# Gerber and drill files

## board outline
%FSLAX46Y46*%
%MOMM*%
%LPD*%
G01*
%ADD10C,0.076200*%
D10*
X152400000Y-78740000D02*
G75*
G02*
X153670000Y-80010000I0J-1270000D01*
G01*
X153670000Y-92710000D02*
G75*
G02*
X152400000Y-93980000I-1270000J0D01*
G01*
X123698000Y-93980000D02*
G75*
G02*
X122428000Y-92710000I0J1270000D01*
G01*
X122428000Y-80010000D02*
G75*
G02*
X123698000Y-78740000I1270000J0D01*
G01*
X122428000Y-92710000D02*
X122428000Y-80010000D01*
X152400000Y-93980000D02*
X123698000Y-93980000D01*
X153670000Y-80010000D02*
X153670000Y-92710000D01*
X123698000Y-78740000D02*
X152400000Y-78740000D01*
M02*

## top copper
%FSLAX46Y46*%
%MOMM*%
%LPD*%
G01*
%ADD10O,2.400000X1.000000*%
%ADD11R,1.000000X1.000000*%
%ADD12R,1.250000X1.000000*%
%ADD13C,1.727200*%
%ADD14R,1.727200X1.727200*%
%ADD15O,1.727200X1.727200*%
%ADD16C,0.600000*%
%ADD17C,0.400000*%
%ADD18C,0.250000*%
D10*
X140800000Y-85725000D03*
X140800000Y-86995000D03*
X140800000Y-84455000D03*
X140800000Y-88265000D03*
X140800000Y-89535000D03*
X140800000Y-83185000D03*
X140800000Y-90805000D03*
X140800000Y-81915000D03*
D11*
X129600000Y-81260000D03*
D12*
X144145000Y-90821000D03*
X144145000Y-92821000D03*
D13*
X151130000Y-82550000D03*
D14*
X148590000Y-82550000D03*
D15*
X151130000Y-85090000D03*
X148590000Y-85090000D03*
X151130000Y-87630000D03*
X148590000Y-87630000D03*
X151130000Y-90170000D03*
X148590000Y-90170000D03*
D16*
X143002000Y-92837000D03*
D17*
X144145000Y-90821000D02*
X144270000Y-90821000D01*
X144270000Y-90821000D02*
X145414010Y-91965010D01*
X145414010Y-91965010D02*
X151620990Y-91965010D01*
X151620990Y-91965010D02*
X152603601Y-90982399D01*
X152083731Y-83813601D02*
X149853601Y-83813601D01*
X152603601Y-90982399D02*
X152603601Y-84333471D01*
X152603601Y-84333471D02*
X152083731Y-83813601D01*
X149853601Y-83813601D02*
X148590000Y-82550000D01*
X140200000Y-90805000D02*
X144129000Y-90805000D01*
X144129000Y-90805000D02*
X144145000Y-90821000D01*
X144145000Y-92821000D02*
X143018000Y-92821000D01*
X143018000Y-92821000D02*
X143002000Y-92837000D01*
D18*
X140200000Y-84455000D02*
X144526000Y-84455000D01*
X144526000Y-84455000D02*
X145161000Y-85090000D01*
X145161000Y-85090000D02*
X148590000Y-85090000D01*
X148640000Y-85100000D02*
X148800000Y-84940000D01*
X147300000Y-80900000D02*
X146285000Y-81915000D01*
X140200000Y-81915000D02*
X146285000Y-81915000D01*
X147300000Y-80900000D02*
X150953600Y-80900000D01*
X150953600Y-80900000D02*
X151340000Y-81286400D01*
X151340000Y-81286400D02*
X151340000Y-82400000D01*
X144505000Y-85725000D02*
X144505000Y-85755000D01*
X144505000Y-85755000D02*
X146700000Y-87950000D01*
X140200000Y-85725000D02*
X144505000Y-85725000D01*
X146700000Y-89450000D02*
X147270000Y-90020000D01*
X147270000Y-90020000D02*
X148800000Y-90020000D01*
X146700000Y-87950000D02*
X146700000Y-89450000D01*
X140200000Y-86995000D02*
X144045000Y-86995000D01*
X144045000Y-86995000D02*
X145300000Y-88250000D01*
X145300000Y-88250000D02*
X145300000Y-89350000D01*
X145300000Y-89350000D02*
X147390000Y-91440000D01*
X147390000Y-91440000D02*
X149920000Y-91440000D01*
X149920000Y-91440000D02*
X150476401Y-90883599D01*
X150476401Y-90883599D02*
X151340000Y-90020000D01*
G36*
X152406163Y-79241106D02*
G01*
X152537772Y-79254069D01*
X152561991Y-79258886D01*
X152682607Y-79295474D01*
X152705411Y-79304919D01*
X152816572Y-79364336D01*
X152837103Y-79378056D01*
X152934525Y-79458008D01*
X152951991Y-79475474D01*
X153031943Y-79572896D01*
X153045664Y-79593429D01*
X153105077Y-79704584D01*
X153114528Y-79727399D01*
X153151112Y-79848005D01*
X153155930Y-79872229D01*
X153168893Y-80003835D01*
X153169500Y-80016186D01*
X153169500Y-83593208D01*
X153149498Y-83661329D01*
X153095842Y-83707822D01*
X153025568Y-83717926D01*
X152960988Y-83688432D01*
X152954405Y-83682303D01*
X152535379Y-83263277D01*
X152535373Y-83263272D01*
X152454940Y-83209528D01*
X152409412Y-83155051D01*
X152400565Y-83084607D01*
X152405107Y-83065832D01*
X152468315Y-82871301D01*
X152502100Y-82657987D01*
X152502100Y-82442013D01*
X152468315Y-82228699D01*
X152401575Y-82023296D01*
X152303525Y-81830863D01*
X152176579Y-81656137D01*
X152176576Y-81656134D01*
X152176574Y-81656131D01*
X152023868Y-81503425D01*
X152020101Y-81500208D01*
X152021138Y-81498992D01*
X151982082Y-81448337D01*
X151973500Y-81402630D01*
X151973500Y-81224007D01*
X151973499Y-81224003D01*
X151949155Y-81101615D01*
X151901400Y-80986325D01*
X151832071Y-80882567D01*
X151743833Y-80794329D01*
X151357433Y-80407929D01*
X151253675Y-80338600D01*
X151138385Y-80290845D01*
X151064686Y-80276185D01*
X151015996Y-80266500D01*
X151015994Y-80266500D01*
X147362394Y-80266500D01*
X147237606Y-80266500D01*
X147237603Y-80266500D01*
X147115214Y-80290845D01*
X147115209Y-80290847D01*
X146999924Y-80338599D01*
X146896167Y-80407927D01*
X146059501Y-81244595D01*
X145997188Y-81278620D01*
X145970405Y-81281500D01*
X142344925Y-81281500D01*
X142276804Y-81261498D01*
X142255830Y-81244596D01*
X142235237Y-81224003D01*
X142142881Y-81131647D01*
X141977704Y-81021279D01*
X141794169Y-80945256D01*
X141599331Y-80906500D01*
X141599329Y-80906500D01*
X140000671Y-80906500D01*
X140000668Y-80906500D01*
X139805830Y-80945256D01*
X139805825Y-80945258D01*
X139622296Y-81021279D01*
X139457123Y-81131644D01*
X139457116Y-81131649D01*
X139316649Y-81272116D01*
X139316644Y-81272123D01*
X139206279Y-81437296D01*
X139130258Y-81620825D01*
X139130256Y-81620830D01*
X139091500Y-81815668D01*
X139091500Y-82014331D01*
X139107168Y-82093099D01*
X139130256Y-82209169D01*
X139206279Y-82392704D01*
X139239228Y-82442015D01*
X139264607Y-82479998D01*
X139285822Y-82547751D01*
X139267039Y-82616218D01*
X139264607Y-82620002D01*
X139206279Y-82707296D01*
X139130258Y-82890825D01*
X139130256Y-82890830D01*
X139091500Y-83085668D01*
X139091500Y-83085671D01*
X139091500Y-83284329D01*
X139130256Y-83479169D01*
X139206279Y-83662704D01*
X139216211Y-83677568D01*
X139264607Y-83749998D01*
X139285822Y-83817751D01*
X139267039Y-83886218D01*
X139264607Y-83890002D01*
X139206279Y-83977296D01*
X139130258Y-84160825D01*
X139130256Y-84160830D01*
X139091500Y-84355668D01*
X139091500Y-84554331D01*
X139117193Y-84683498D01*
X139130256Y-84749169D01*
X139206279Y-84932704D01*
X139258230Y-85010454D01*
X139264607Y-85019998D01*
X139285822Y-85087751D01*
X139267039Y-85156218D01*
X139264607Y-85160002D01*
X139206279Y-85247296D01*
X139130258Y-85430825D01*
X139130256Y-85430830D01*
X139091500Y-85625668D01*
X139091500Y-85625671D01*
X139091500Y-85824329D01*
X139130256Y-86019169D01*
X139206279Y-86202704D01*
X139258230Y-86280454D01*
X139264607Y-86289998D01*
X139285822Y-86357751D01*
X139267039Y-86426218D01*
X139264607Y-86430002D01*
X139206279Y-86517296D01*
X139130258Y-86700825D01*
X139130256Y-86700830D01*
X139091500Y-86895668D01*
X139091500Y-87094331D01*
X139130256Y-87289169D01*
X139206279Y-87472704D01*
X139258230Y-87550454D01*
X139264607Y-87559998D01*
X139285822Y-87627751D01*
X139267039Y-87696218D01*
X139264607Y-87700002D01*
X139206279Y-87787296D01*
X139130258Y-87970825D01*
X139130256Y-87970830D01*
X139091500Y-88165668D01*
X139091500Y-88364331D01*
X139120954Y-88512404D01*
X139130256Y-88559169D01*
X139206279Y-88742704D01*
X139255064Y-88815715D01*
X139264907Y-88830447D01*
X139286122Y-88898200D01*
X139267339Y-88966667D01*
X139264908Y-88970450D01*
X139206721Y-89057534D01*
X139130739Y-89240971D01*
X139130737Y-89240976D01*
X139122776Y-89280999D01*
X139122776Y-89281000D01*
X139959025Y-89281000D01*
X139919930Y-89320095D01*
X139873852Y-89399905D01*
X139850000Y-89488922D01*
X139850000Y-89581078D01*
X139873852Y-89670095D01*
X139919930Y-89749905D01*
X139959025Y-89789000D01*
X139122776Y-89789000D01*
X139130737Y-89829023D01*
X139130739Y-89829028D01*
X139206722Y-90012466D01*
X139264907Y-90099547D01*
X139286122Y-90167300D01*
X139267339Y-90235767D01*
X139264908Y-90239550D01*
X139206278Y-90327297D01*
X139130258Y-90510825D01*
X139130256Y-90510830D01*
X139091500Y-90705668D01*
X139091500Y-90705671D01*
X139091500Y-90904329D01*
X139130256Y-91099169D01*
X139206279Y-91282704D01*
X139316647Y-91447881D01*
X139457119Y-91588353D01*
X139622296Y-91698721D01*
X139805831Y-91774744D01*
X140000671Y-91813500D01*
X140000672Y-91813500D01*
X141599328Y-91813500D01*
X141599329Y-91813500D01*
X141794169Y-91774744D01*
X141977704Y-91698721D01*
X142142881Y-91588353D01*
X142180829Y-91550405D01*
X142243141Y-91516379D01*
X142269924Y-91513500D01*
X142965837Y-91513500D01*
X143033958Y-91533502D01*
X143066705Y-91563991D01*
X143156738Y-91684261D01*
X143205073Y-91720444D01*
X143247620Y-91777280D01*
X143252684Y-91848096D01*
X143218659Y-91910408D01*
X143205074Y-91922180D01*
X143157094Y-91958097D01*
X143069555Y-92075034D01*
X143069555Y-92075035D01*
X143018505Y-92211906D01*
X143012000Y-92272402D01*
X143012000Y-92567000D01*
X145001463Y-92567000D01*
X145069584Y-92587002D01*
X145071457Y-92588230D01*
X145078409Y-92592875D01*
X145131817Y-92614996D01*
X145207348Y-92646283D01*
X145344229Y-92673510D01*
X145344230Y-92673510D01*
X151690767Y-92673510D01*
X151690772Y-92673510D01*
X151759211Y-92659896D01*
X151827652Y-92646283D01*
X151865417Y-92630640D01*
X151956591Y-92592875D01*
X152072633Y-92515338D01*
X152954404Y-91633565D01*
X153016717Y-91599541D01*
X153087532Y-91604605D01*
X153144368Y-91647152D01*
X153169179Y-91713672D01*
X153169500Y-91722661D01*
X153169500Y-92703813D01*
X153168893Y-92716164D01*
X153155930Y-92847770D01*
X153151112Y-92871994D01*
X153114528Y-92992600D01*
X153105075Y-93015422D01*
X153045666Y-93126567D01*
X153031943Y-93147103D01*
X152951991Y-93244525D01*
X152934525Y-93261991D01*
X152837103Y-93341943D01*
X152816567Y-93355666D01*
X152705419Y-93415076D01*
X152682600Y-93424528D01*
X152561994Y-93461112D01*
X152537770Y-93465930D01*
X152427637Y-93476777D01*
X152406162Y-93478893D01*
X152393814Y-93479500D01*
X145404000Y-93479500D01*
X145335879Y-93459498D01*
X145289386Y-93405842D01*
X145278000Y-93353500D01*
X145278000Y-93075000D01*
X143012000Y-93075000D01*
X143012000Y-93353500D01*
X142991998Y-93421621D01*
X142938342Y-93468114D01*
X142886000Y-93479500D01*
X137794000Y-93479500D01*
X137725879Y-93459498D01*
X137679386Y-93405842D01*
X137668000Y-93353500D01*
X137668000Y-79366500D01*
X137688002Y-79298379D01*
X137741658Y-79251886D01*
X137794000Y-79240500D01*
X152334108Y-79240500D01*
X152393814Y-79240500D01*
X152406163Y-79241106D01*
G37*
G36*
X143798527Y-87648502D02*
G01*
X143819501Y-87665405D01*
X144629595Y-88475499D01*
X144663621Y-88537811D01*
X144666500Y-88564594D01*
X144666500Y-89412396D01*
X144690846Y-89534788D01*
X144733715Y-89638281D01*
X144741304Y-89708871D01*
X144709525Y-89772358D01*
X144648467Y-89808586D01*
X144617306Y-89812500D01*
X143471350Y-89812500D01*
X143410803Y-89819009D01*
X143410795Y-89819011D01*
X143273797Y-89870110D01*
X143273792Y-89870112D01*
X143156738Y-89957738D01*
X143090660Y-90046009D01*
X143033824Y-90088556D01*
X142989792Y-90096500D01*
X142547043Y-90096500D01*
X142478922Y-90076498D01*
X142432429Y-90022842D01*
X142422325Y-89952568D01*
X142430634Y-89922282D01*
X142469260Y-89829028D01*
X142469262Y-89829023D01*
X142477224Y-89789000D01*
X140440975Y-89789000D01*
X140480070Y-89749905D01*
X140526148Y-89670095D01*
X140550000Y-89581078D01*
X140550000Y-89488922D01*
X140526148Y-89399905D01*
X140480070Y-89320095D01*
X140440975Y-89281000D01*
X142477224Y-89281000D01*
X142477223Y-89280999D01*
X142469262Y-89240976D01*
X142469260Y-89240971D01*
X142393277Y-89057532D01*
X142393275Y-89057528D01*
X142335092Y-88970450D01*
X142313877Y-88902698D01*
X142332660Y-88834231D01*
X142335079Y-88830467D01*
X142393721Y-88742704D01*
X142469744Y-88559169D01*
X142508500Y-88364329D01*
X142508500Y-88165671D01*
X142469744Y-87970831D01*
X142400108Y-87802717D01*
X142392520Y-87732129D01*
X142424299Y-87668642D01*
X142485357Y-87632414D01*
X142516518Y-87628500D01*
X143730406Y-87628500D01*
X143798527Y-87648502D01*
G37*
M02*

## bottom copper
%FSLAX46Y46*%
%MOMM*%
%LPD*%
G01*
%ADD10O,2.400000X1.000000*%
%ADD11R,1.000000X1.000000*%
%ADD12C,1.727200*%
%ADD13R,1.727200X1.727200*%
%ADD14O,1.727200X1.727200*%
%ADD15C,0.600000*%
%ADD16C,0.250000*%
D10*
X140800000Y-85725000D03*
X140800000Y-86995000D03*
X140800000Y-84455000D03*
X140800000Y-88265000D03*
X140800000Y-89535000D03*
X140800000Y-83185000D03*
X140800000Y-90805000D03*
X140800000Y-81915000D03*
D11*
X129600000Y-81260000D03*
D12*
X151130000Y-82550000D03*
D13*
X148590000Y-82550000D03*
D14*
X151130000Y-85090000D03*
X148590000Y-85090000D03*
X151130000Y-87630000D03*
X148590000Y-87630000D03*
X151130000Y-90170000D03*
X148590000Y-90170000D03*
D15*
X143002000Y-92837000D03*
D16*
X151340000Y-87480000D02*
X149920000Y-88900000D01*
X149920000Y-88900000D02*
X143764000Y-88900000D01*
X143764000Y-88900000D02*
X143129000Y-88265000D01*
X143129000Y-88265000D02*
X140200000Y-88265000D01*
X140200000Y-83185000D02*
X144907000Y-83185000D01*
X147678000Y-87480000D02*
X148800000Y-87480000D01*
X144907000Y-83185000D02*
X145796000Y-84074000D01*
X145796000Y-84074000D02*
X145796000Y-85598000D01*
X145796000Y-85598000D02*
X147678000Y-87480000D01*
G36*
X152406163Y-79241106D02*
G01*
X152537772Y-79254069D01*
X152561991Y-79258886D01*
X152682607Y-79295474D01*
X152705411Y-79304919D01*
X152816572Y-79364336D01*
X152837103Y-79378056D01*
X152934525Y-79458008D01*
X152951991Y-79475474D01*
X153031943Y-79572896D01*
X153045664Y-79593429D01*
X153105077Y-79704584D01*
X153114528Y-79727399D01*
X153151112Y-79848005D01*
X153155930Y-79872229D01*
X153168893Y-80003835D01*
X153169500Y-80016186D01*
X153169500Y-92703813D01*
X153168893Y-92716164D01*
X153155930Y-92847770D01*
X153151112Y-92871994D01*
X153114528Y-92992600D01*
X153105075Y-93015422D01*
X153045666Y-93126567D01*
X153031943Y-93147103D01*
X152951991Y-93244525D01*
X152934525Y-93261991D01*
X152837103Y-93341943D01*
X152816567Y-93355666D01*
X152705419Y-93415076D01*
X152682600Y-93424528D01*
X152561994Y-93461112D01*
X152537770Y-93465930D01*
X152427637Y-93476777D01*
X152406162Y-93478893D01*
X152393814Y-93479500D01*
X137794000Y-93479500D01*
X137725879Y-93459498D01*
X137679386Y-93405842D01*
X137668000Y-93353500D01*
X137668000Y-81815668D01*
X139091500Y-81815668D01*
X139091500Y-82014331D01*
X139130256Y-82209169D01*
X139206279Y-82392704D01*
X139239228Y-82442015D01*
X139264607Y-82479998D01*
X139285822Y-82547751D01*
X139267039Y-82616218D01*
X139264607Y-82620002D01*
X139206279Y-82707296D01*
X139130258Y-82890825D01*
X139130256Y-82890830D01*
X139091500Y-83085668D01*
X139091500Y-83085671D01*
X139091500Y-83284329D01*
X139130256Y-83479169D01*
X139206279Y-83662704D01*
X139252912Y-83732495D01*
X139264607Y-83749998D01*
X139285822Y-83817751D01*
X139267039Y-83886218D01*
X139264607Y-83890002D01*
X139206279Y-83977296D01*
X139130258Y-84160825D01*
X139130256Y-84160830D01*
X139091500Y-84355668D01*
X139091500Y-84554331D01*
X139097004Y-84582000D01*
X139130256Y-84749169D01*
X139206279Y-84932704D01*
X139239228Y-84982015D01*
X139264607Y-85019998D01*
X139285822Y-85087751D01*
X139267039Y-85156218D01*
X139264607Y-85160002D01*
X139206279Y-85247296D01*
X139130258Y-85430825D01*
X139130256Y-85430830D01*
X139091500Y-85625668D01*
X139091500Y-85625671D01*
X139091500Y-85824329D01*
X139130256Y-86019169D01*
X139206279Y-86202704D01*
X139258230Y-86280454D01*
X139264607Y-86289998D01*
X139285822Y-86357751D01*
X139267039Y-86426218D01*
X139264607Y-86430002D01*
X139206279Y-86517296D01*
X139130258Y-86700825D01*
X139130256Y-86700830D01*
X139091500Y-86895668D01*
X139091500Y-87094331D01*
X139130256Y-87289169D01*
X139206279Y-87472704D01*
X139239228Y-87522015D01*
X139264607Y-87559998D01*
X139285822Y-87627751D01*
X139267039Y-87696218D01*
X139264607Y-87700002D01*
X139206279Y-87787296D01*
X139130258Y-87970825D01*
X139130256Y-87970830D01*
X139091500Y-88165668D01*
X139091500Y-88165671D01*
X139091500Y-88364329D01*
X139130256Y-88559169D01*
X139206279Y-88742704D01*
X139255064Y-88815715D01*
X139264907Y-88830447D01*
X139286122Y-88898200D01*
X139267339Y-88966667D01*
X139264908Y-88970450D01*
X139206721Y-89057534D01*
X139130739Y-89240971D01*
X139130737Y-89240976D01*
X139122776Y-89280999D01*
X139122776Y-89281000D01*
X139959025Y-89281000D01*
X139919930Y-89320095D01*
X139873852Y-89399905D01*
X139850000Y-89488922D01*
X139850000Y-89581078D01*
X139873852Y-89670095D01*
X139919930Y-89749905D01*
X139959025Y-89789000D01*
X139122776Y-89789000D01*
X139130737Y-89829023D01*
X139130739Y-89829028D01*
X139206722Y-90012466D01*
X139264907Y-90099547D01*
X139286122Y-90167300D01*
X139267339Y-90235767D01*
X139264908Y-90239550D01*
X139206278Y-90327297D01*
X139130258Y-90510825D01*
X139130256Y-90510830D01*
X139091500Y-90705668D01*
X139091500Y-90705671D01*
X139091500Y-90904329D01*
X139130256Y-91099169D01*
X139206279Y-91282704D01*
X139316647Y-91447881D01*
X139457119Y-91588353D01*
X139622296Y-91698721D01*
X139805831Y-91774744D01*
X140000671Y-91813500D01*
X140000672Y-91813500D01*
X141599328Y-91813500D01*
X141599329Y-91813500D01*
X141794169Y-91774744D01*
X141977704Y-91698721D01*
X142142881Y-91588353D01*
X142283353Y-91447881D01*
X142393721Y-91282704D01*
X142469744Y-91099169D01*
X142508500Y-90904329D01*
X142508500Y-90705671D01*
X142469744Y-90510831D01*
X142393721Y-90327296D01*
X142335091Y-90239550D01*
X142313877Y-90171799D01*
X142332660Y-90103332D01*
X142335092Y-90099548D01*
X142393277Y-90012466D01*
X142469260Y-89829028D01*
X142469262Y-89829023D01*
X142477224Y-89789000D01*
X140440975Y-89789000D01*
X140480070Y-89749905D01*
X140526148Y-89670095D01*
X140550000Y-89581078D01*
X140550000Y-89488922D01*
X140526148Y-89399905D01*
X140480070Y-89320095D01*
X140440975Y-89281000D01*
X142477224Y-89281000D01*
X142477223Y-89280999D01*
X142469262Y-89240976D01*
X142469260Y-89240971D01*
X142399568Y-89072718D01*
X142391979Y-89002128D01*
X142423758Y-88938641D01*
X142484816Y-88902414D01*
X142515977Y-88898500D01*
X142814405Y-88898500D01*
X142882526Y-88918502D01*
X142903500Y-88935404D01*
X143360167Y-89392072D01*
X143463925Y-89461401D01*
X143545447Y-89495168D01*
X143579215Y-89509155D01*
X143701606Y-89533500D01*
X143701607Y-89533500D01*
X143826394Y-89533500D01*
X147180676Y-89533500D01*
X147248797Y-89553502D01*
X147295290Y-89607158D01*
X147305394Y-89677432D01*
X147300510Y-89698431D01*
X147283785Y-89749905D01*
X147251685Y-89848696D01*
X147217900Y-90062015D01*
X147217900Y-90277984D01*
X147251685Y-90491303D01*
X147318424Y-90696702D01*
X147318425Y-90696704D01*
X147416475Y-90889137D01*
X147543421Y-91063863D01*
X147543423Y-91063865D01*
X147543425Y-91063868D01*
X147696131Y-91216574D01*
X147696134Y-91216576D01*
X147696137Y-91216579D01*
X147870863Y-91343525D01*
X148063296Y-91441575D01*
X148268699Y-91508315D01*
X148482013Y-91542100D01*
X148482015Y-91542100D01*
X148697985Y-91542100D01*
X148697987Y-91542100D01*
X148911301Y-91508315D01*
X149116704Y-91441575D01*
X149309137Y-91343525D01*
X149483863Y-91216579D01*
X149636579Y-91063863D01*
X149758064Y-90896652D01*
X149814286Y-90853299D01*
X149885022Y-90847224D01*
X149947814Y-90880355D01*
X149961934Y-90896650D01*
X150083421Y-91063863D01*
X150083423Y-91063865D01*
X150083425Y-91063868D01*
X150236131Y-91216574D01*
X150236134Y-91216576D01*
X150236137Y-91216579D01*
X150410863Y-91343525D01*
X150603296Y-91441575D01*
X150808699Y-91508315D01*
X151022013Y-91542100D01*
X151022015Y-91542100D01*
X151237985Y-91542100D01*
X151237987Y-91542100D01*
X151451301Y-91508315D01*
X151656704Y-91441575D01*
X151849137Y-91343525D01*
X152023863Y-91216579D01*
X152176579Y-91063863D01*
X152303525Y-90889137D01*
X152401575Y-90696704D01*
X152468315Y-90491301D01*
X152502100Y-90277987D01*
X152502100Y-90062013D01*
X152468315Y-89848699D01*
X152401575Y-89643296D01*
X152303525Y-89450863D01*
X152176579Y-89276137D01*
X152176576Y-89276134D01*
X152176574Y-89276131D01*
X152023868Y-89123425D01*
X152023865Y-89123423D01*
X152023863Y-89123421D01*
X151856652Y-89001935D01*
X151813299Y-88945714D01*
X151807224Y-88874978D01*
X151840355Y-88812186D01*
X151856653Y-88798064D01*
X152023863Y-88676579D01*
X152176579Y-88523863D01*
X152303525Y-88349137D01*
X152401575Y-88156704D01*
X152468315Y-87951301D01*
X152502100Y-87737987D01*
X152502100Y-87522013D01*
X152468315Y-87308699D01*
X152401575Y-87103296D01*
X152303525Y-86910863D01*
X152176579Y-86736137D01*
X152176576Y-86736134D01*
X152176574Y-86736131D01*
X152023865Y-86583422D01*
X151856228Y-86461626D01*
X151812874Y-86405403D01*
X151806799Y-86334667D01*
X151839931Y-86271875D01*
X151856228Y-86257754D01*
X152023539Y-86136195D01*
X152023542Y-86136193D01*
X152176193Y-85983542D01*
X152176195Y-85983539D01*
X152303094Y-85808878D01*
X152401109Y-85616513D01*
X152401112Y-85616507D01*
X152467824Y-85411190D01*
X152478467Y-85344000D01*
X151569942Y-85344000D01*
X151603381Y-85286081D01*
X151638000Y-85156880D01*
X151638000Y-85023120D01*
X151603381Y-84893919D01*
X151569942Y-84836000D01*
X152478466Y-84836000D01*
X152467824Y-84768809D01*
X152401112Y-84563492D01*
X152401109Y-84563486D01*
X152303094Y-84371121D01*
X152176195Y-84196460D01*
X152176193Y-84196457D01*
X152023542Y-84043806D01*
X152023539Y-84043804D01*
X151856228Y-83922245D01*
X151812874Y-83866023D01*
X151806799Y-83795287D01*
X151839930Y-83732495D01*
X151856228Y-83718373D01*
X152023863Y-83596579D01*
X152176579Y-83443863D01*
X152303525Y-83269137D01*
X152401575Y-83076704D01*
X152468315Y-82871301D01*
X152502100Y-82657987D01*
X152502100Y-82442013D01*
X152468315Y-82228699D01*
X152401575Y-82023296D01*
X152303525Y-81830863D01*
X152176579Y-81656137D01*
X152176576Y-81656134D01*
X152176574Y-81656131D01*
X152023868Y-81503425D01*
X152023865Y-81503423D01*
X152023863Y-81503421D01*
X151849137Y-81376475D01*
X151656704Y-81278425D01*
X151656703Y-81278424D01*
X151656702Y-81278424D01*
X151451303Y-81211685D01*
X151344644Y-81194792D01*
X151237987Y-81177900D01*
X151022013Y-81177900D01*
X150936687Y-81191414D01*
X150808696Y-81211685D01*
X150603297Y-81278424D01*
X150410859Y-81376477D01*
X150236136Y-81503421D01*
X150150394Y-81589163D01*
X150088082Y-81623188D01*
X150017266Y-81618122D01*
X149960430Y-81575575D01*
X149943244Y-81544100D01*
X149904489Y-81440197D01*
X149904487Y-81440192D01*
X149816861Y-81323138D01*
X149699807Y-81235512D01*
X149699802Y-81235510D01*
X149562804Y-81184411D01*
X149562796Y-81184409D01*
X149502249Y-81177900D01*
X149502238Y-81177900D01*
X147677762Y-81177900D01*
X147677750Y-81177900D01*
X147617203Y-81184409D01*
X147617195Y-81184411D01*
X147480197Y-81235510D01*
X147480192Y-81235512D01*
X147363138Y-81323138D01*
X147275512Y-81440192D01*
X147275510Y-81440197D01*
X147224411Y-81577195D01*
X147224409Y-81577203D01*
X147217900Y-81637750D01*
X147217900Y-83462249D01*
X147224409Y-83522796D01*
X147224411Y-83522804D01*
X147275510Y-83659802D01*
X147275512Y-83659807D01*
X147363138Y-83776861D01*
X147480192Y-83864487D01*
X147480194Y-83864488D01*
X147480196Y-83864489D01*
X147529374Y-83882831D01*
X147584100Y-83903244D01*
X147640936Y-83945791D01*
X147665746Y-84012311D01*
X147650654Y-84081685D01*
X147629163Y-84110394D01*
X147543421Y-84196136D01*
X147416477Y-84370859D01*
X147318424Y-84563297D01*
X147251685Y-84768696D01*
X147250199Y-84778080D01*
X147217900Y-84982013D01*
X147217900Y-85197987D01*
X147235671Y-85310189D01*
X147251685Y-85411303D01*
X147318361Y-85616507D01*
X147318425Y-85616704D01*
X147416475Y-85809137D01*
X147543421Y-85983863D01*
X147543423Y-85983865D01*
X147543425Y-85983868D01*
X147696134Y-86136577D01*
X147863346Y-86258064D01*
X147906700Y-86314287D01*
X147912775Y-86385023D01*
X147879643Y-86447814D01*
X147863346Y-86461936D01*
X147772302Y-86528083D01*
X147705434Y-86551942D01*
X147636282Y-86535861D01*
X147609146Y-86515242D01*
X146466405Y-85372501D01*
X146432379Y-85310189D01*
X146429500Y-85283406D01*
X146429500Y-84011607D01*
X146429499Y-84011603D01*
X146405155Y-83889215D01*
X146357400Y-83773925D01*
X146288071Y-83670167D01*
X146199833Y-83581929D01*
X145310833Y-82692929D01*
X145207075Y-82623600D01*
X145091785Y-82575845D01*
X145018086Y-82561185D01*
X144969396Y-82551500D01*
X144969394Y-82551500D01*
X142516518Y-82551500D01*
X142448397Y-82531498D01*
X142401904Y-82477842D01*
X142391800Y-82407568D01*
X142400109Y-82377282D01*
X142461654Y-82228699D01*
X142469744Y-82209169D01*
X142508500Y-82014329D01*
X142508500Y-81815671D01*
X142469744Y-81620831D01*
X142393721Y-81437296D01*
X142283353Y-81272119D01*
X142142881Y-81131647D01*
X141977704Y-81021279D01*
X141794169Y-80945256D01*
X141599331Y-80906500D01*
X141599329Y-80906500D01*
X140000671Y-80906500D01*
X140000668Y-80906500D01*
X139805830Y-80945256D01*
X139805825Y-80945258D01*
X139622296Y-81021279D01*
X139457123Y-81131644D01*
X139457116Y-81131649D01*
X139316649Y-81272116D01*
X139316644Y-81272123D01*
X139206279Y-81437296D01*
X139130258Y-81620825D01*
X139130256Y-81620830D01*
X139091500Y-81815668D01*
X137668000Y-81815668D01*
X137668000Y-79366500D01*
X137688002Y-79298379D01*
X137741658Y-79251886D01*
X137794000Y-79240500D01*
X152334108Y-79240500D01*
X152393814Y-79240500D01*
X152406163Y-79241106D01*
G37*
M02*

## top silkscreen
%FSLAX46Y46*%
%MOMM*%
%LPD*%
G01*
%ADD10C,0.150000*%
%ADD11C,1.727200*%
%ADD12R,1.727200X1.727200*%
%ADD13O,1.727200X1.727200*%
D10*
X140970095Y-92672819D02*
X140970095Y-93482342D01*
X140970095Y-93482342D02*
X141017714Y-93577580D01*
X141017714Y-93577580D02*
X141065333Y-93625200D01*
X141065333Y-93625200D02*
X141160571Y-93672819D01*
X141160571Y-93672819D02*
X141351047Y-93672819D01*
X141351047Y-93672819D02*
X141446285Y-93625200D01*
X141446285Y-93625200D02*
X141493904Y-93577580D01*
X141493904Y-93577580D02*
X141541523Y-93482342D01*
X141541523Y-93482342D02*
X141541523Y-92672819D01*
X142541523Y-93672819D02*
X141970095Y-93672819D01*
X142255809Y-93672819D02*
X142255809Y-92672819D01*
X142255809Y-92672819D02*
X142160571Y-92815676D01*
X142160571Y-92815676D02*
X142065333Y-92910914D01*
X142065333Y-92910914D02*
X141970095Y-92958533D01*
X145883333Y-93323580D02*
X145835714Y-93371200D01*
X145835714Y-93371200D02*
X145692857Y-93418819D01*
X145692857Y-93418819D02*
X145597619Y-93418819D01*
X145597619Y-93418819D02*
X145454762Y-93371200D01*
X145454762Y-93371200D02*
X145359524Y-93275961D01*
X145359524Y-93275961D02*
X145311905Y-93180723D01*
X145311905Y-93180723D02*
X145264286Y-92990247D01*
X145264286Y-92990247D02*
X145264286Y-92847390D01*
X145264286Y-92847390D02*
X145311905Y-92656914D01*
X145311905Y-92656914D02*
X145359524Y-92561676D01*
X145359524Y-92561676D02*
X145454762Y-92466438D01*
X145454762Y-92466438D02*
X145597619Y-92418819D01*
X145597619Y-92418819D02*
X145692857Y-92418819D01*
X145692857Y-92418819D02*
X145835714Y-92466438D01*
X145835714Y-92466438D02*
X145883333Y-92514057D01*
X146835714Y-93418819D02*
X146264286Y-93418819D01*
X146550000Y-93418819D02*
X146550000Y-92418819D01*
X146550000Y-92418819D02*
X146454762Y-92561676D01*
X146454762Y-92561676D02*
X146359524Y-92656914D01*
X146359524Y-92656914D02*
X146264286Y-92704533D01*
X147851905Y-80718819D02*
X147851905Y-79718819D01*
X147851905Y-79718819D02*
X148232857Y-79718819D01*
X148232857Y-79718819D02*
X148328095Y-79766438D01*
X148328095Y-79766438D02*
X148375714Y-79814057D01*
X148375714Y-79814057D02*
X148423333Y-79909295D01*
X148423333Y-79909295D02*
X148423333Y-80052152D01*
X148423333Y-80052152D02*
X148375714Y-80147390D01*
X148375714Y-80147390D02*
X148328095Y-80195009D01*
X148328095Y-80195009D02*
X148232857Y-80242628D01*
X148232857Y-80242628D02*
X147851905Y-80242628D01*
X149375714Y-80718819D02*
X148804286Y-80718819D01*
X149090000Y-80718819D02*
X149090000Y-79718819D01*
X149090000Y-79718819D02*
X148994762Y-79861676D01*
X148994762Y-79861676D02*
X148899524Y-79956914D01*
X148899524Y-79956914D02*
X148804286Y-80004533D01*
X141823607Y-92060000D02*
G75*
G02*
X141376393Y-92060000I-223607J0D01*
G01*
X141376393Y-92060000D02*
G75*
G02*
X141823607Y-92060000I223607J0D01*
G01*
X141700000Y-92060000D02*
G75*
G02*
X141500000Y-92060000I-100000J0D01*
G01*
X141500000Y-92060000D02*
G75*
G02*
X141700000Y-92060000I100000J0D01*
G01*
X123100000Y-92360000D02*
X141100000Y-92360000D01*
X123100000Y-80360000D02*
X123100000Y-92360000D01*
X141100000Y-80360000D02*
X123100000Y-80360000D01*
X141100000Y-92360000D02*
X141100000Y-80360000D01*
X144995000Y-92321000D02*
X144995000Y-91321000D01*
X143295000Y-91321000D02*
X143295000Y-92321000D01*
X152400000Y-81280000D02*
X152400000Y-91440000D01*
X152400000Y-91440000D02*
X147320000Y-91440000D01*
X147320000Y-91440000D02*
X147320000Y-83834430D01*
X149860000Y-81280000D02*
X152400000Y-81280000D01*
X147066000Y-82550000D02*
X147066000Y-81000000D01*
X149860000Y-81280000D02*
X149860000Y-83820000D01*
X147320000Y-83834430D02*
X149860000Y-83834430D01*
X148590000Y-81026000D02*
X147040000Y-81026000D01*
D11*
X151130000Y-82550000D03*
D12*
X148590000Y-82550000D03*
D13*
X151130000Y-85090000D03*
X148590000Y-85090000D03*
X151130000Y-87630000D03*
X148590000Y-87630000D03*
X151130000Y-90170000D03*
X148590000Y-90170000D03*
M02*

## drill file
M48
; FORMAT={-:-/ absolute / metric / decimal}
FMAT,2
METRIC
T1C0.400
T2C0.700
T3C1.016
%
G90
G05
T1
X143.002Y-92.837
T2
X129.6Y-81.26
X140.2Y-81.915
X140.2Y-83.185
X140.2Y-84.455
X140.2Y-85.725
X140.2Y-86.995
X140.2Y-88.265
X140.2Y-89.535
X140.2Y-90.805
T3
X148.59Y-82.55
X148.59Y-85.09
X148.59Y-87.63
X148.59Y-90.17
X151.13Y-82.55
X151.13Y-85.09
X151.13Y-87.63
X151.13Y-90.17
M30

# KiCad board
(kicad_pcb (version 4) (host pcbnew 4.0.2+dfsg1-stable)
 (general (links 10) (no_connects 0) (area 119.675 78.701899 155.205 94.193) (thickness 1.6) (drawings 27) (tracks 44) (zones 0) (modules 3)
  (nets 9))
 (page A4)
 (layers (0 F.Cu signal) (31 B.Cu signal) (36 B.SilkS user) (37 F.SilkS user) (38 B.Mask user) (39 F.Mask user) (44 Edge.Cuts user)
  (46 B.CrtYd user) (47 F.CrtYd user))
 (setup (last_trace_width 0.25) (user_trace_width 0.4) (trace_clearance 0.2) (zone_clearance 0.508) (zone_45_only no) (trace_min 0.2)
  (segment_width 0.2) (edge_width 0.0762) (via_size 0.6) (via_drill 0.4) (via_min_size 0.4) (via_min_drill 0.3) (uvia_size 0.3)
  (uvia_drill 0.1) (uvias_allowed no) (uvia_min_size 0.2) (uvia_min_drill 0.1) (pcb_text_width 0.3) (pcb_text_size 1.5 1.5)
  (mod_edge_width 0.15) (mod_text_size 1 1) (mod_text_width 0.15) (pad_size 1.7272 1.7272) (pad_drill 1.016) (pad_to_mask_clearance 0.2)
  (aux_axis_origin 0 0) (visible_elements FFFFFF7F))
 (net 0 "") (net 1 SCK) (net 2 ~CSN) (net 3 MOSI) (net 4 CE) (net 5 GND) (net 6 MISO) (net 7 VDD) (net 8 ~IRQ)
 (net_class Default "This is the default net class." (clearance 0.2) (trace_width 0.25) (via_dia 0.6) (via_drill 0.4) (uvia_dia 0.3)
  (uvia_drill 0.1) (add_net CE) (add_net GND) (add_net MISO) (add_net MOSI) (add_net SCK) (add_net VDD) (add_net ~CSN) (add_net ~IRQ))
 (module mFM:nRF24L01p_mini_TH (layer F.Cu) (at 141.1 86.36 90)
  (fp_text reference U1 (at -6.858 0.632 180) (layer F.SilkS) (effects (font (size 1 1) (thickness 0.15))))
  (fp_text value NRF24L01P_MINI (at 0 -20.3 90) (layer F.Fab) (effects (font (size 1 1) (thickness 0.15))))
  (fp_circle (center -5.7 0.5) (end -5.6 0.7) (layer F.SilkS) (width 0.15))
  (fp_circle (center -5.7 0.5) (end -5.6 0.5) (layer F.SilkS) (width 0.15))
  (fp_line (start -6 -18) (end -6 0) (layer F.SilkS) (width 0.15))
  (fp_line (start 6 -18) (end -6 -18) (layer F.SilkS) (width 0.15))
  (fp_line (start 6 0) (end 6 -18) (layer F.SilkS) (width 0.15))
  (fp_line (start -6 0) (end 6 0) (layer F.SilkS) (width 0.15))
  (pad 5 thru_hole oval (at 0.635 -0.9 90) (size 1 2.4) (drill 0.7 (offset 0 0.6)) (layers *.Cu *.Mask) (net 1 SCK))
  (pad 4 thru_hole oval (at -0.635 -0.9 90) (size 1 2.4) (drill 0.7 (offset 0 0.6)) (layers *.Cu *.Mask) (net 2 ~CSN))
  (pad 6 thru_hole oval (at 1.905 -0.9 90) (size 1 2.4) (drill 0.7 (offset 0 0.6)) (layers *.Cu *.Mask) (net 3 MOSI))
  (pad 3 thru_hole oval (at -1.905 -0.9 90) (size 1 2.4) (drill 0.7 (offset 0 0.6)) (layers *.Cu *.Mask) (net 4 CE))
  (pad 2 thru_hole oval (at -3.175 -0.9 90) (size 1 2.4) (drill 0.7 (offset 0 0.6)) (layers *.Cu *.Mask) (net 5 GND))
  (pad 7 thru_hole oval (at 3.175 -0.9 90) (size 1 2.4) (drill 0.7 (offset 0 0.6)) (layers *.Cu *.Mask) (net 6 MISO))
  (pad 1 thru_hole oval (at -4.445 -0.9 90) (size 1 2.4) (drill 0.7 (offset 0 0.6)) (layers *.Cu *.Mask) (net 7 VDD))
  (pad 8 thru_hole oval (at 4.445 -0.9 90) (size 1 2.4) (drill 0.7 (offset 0 0.6)) (layers *.Cu *.Mask) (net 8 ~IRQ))
  (pad 9 thru_hole rect (at 5.1 -11.5 180) (size 1 1) (drill 0.7) (layers *.Cu *.Mask)))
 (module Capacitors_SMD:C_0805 (layer F.Cu) (at 144.145 91.821 270)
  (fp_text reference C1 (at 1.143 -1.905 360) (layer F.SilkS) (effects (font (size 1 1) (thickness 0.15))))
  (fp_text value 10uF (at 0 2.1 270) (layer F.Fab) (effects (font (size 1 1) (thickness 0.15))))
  (fp_line (start 0.5 -0.85) (end -0.5 -0.85) (layer F.SilkS) (width 0.15))
  (fp_line (start -0.5 0.85) (end 0.5 0.85) (layer F.SilkS) (width 0.15))
  (pad 1 smd rect (at -1 0 270) (size 1 1.25) (layers F.Cu F.Mask) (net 7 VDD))
  (pad 2 smd rect (at 1 0 270) (size 1 1.25) (layers F.Cu F.Mask) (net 5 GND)))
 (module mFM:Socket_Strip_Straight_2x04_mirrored (layer F.Cu) (at 151.13 82.55 270)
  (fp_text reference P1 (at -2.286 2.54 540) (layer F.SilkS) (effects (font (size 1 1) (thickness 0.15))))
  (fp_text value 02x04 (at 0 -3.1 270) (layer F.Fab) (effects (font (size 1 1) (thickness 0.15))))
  (fp_line (start -1.27 -1.27) (end 8.89 -1.27) (layer F.SilkS) (width 0.15))
  (fp_line (start 8.89 -1.27) (end 8.89 3.81) (layer F.SilkS) (width 0.15))
  (fp_line (start 8.89 3.81) (end 1.28443 3.81) (layer F.SilkS) (width 0.15))
  (fp_line (start -1.27 1.27) (end -1.27 -1.27) (layer F.SilkS) (width 0.15))
  (fp_line (start 0 4.064) (end -1.55 4.064) (layer F.SilkS) (width 0.15))
  (fp_line (start -1.27 1.27) (end 1.27 1.27) (layer F.SilkS) (width 0.15))
  (fp_line (start 1.28443 3.81) (end 1.28443 1.27) (layer F.SilkS) (width 0.15))
  (fp_line (start -1.524 2.54) (end -1.524 4.09) (layer F.SilkS) (width 0.15))
  (pad 2 thru_hole circle (at 0 0 270) (size 1.7272 1.7272) (drill 1.016) (layers *.Cu *.Mask F.SilkS) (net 8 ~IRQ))
  (pad 1 thru_hole rect (at 0 2.54 270) (size 1.7272 1.7272) (drill 1.016) (layers *.Cu *.Mask F.SilkS) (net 7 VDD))
  (pad 4 thru_hole oval (at 2.54 0 270) (size 1.7272 1.7272) (drill 1.016) (layers *.Cu *.Mask F.SilkS) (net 5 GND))
  (pad 3 thru_hole oval (at 2.54 2.54 270) (size 1.7272 1.7272) (drill 1.016) (layers *.Cu *.Mask F.SilkS) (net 3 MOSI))
  (pad 6 thru_hole oval (at 5.08 0 270) (size 1.7272 1.7272) (drill 1.016) (layers *.Cu *.Mask F.SilkS) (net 4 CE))
  (pad 5 thru_hole oval (at 5.08 2.54 270) (size 1.7272 1.7272) (drill 1.016) (layers *.Cu *.Mask F.SilkS) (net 6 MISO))
  (pad 8 thru_hole oval (at 7.62 0 270) (size 1.7272 1.7272) (drill 1.016) (layers *.Cu *.Mask F.SilkS) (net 2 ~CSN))
  (pad 7 thru_hole oval (at 7.62 2.54 270) (size 1.7272 1.7272) (drill 1.016) (layers *.Cu *.Mask F.SilkS) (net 1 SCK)))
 (gr_arc (start 152.4 80.01) (end 152.4 78.74) (angle 90) (layer Edge.Cuts) (width 0.0762))
 (gr_arc (start 152.4 92.71) (end 153.67 92.71) (angle 90) (layer Edge.Cuts) (width 0.0762))
 (gr_arc (start 123.698 92.71) (end 123.698 93.98) (angle 90) (layer Edge.Cuts) (width 0.0762))
 (gr_arc (start 123.698 80.01) (end 122.428 80.01) (angle 90) (layer Edge.Cuts) (width 0.0762))
 (gr_line (start 122.428 92.71) (end 122.428 80.01) (layer Edge.Cuts) (width 0.0762))
 (gr_line (start 152.4 93.98) (end 123.698 93.98) (layer Edge.Cuts) (width 0.0762))
 (gr_line (start 153.67 80.01) (end 153.67 92.71) (layer Edge.Cuts) (width 0.0762))
 (gr_line (start 123.698 78.74) (end 152.4 78.74) (layer Edge.Cuts) (width 0.0762))
 (segment (start 144.145 90.821) (end 144.27 90.821) (width 0.4) (layer F.Cu) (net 7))
 (segment (start 144.27 90.821) (end 145.41401 91.96501) (width 0.4) (layer F.Cu) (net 7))
 (segment (start 145.41401 91.96501) (end 151.62099 91.96501) (width 0.4) (layer F.Cu) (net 7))
 (segment (start 151.62099 91.96501) (end 152.603601 90.982399) (width 0.4) (layer F.Cu) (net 7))
 (segment (start 152.083731 83.813601) (end 149.853601 83.813601) (width 0.4) (layer F.Cu) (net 7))
 (segment (start 152.603601 90.982399) (end 152.603601 84.333471) (width 0.4) (layer F.Cu) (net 7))
 (segment (start 152.603601 84.333471) (end 152.083731 83.813601) (width 0.4) (layer F.Cu) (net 7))
 (segment (start 149.853601 83.813601) (end 148.59 82.55) (width 0.4) (layer F.Cu) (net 7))
 (segment (start 140.2 90.805) (end 144.129 90.805) (width 0.4) (layer F.Cu) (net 7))
 (segment (start 144.129 90.805) (end 144.145 90.821) (width 0.4) (layer F.Cu) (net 7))
 (segment (start 144.145 92.821) (end 143.018 92.821) (width 0.4) (layer F.Cu) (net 5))
 (segment (start 143.018 92.821) (end 143.002 92.837) (width 0.4) (layer F.Cu) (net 5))
 (via (at 143.002 92.837) (size 0.6) (drill 0.4) (layers F.Cu B.Cu) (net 5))
 (segment (start 151.34 87.48) (end 149.92 88.9) (width 0.25) (layer B.Cu) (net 4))
 (segment (start 149.92 88.9) (end 143.764 88.9) (width 0.25) (layer B.Cu) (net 4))
 (segment (start 143.764 88.9) (end 143.129 88.265) (width 0.25) (layer B.Cu) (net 4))
 (segment (start 143.129 88.265) (end 140.2 88.265) (width 0.25) (layer B.Cu) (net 4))
 (segment (start 140.2 84.455) (end 144.526 84.455) (width 0.25) (layer F.Cu) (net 3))
 (segment (start 144.526 84.455) (end 145.161 85.09) (width 0.25) (layer F.Cu) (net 3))
 (segment (start 145.161 85.09) (end 148.59 85.09) (width 0.25) (layer F.Cu) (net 3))
 (segment (start 148.64 85.1) (end 148.8 84.94) (width 0.25) (layer F.Cu) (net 3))
 (segment (start 140.2 83.185) (end 144.907 83.185) (width 0.25) (layer B.Cu) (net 6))
 (segment (start 147.678 87.48) (end 148.8 87.48) (width 0.25) (layer B.Cu) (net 6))
 (segment (start 144.907 83.185) (end 145.796 84.074) (width 0.25) (layer B.Cu) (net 6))
 (segment (start 145.796 84.074) (end 145.796 85.598) (width 0.25) (layer B.Cu) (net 6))
 (segment (start 145.796 85.598) (end 147.678 87.48) (width 0.25) (layer B.Cu) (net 6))
 (segment (start 147.3 80.9) (end 146.285 81.915) (width 0.25) (layer F.Cu) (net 8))
 (segment (start 140.2 81.915) (end 146.285 81.915) (width 0.25) (layer F.Cu) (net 8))
 (segment (start 147.3 80.9) (end 150.9536 80.9) (width 0.25) (layer F.Cu) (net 8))
 (segment (start 150.9536 80.9) (end 151.34 81.2864) (width 0.25) (layer F.Cu) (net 8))
 (segment (start 151.34 81.2864) (end 151.34 82.4) (width 0.25) (layer F.Cu) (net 8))
 (segment (start 144.505 85.725) (end 144.505 85.755) (width 0.25) (layer F.Cu) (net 1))
 (segment (start 144.505 85.755) (end 146.7 87.95) (width 0.25) (layer F.Cu) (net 1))
 (segment (start 140.2 85.725) (end 144.505 85.725) (width 0.25) (layer F.Cu) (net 1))
 (segment (start 146.7 89.45) (end 147.27 90.02) (width 0.25) (layer F.Cu) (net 1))
 (segment (start 147.27 90.02) (end 148.8 90.02) (width 0.25) (layer F.Cu) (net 1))
 (segment (start 146.7 87.95) (end 146.7 89.45) (width 0.25) (layer F.Cu) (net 1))
 (segment (start 140.2 86.995) (end 144.045 86.995) (width 0.25) (layer F.Cu) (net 2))
 (segment (start 144.045 86.995) (end 145.3 88.25) (width 0.25) (layer F.Cu) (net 2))
 (segment (start 145.3 88.25) (end 145.3 89.35) (width 0.25) (layer F.Cu) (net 2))
 (segment (start 145.3 89.35) (end 147.39 91.44) (width 0.25) (layer F.Cu) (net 2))
 (segment (start 147.39 91.44) (end 149.92 91.44) (width 0.25) (layer F.Cu) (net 2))
 (segment (start 149.92 91.44) (end 150.476401 90.883599) (width 0.25) (layer F.Cu) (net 2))
 (segment (start 150.476401 90.883599) (end 151.34 90.02) (width 0.25) (layer F.Cu) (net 2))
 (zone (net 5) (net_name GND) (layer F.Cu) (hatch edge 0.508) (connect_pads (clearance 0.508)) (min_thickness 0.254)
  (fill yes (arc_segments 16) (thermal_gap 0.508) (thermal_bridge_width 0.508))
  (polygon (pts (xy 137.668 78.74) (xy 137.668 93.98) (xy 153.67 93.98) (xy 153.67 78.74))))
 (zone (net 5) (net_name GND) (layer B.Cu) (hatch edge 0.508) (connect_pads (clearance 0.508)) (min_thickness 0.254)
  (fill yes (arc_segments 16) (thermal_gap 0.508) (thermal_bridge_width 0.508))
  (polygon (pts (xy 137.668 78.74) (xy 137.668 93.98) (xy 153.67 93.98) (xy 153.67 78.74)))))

